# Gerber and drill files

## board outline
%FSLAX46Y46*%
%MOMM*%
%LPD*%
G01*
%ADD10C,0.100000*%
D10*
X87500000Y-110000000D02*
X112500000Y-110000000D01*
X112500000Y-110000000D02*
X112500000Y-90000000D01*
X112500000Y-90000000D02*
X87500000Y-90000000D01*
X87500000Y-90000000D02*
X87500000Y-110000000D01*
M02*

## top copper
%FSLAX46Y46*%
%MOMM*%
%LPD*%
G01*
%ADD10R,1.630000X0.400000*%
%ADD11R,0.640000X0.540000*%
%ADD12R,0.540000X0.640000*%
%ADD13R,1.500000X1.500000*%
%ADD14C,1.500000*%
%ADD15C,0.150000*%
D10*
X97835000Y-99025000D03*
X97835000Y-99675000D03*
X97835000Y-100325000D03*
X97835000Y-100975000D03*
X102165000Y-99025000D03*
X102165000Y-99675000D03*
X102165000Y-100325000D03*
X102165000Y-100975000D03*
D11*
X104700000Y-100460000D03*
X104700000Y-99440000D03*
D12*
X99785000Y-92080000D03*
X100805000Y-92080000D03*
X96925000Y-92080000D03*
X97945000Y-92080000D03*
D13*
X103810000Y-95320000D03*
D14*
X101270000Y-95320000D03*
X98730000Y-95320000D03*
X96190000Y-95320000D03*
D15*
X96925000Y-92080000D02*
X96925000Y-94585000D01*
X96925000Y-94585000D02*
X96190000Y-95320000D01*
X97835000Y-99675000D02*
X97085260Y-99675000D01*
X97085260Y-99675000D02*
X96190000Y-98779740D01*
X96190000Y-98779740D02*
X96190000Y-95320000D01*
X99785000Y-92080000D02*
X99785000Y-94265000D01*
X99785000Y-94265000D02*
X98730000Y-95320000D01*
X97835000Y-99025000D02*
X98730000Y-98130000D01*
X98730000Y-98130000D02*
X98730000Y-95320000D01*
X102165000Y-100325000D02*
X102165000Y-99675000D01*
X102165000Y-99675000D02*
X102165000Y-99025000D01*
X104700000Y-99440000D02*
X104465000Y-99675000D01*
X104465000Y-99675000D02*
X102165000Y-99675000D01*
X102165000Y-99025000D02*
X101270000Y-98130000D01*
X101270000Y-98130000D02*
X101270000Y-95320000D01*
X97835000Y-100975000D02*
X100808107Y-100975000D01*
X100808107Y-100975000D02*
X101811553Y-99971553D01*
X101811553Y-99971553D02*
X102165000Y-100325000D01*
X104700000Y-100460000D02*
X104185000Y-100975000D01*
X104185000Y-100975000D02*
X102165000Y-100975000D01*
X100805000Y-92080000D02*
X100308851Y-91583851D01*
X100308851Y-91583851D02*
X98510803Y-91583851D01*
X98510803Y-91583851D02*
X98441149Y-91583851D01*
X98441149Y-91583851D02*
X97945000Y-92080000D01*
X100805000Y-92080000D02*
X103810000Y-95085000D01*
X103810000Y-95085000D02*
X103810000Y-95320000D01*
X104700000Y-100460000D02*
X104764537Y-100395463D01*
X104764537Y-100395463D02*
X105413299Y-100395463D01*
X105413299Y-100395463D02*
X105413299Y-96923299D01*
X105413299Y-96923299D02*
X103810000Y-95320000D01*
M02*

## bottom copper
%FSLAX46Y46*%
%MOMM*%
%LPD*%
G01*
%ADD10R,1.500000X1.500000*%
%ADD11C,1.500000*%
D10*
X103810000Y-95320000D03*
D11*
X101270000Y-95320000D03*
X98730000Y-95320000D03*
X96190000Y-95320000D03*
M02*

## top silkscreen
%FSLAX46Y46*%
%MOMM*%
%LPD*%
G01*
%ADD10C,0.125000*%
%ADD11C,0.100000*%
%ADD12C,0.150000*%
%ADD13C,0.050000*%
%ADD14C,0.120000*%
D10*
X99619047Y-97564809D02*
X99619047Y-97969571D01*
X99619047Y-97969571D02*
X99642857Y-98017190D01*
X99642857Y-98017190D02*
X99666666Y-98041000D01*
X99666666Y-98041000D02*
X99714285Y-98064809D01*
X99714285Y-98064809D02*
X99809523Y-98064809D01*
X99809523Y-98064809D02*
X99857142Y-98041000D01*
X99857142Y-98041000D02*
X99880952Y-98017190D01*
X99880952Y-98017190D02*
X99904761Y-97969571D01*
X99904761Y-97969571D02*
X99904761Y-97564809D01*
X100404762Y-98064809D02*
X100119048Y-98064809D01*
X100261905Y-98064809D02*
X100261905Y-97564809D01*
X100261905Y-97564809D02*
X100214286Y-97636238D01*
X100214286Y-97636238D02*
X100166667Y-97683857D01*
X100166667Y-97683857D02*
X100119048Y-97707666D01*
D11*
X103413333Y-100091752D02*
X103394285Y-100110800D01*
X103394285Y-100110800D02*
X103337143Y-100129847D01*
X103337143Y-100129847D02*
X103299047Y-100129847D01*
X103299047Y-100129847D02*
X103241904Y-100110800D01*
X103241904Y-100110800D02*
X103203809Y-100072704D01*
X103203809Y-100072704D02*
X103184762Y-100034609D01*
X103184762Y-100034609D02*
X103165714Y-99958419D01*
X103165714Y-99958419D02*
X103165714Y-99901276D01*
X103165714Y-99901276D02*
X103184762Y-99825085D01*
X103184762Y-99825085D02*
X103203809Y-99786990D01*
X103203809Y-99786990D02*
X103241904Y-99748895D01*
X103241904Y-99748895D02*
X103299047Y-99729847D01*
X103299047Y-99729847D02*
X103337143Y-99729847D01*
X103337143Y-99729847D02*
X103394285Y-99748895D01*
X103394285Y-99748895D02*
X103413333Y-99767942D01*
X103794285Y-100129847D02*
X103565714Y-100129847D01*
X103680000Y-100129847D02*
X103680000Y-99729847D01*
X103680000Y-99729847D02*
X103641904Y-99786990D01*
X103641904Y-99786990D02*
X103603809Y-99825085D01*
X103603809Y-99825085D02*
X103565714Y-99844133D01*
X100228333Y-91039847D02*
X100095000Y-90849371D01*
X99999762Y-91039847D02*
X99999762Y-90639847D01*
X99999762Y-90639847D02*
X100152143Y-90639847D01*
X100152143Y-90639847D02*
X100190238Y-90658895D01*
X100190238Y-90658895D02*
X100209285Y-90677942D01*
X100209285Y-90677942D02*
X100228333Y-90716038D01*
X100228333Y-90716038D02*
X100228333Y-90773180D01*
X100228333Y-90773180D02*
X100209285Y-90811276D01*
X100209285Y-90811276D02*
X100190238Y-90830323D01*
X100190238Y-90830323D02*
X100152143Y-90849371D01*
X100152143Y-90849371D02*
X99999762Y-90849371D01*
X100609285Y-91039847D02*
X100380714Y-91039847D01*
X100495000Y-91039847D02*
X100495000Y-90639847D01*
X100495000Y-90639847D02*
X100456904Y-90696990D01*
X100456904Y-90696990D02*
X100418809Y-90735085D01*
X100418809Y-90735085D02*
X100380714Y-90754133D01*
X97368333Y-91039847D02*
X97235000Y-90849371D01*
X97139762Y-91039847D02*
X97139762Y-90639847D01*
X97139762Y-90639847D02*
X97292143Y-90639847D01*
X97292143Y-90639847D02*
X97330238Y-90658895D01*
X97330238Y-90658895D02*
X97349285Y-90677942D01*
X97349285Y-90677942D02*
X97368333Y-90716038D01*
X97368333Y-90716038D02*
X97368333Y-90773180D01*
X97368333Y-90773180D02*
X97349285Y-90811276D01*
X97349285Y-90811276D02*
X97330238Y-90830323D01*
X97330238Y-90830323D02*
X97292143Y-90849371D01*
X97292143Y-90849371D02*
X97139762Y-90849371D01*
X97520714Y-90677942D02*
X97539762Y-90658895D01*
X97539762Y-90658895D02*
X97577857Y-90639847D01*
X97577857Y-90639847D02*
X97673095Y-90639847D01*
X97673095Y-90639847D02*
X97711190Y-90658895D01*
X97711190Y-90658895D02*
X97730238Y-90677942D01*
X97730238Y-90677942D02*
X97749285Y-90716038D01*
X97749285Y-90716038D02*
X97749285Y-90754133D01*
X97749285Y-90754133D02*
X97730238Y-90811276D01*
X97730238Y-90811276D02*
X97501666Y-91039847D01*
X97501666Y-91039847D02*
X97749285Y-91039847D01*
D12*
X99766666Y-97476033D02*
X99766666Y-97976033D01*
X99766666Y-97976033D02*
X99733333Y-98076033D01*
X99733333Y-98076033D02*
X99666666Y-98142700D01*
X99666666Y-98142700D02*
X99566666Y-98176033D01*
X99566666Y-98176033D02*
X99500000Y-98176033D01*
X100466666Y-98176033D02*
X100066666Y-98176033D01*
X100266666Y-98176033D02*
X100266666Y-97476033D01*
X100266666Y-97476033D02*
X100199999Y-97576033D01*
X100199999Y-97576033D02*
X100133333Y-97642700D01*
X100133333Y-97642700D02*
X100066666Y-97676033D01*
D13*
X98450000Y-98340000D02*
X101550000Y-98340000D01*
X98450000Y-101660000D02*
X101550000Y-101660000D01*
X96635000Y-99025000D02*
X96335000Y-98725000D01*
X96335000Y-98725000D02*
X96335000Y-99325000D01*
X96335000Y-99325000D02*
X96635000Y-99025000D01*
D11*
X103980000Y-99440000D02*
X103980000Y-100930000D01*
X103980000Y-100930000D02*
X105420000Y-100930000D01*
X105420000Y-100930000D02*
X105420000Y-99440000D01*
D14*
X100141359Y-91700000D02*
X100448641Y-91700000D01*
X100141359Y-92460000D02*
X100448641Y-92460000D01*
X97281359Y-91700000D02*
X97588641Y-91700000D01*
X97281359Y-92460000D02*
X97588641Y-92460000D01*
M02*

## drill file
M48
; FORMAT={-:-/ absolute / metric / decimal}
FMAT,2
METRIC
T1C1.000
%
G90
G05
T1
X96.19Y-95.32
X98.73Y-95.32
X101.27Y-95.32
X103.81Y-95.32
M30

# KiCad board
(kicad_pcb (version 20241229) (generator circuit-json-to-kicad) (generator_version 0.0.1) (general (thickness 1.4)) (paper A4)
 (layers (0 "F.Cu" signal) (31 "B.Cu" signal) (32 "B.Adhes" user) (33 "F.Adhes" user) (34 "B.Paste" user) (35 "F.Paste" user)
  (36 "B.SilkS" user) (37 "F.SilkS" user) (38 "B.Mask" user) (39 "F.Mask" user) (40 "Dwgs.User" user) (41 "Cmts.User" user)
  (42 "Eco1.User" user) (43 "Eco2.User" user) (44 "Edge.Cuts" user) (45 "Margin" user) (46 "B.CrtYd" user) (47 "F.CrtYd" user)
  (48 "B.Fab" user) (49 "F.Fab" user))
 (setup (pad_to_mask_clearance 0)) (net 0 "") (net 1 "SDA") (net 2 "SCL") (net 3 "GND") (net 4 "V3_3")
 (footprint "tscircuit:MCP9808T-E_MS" (layer F.Cu) (at 100 100 0)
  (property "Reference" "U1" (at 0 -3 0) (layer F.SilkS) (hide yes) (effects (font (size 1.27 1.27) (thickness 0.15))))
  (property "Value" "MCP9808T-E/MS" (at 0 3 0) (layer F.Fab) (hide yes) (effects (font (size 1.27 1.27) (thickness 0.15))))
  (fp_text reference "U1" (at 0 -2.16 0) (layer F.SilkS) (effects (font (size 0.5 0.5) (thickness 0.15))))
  (fp_line (start -1.55 -1.66) (end 1.55 -1.66) (stroke (width 0.05) (type default)) (layer F.SilkS))
  (fp_line (start -1.55 1.66) (end 1.55 1.66) (stroke (width 0.05) (type default)) (layer F.SilkS))
  (fp_line (start -3.3649999999999998 -0.9750000000000001) (end -3.665 -1.2750000000000001) (stroke (width 0.05) (type default))
   (layer F.SilkS))
  (fp_line (start -3.665 -1.2750000000000001) (end -3.665 -0.675) (stroke (width 0.05) (type default)) (layer F.SilkS))
  (fp_line (start -3.665 -0.675) (end -3.3649999999999998 -0.9750000000000001) (stroke (width 0.05) (type default)) (layer F.SilkS))
  (pad "1" smd rect (at -2.165 -0.9750000000000001 0) (size 1.63 0.4) (layers F.Cu F.Paste F.Mask) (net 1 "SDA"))
  (pad "2" smd rect (at -2.165 -0.325 0) (size 1.63 0.4) (layers F.Cu F.Paste F.Mask) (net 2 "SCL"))
  (pad "3" smd rect (at -2.165 0.325 0) (size 1.63 0.4) (layers F.Cu F.Paste F.Mask))
  (pad "4" smd rect (at -2.165 0.9750000000000001 0) (size 1.63 0.4) (layers F.Cu F.Paste F.Mask) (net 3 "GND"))
  (pad "5" smd rect (at 2.165 -0.9750000000000001 0) (size 1.63 0.4) (layers F.Cu F.Paste F.Mask) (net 3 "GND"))
  (pad "6" smd rect (at 2.165 -0.325 0) (size 1.63 0.4) (layers F.Cu F.Paste F.Mask) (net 3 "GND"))
  (pad "7" smd rect (at 2.165 0.325 0) (size 1.63 0.4) (layers F.Cu F.Paste F.Mask) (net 3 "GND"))
  (pad "8" smd rect (at 2.165 0.9750000000000001 0) (size 1.63 0.4) (layers F.Cu F.Paste F.Mask) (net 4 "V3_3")))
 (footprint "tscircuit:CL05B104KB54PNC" (layer F.Cu) (at 104.7 99.95 90)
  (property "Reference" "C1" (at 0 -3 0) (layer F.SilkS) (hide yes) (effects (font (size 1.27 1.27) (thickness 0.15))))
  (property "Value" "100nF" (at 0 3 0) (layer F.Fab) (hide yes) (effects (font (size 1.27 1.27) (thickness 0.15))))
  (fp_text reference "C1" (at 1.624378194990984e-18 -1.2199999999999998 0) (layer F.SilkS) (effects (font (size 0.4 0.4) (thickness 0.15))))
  (fp_line (start 0.51 -0.7199999999999998) (end -0.98 -0.7200000000000001) (stroke (width 0.1) (type default)) (layer F.SilkS))
  (fp_line (start -0.98 -0.7200000000000001) (end -0.98 0.7199999999999999) (stroke (width 0.1) (type default)) (layer F.SilkS))
  (fp_line (start -0.98 0.7199999999999999) (end 0.51 0.7199999999999998) (stroke (width 0.1) (type default)) (layer F.SilkS))
  (pad "1" smd rect (at -0.51 0 0) (size 0.64 0.54) (layers F.Cu F.Paste F.Mask) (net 4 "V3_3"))
  (pad "2" smd rect (at 0.51 0 0) (size 0.64 0.54) (layers F.Cu F.Paste F.Mask) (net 3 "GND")))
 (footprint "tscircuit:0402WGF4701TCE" (layer F.Cu) (at 100.295 92.08 0)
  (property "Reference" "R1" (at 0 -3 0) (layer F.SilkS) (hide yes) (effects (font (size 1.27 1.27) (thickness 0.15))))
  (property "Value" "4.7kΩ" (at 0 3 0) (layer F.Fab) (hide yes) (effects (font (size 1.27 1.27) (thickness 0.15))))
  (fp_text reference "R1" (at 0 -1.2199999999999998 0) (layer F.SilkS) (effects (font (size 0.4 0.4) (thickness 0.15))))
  (fp_line (start -0.153641 -0.3799999999999999) (end 0.15364100000000003 -0.3799999999999999) (stroke (width 0.12) (type default))
   (layer F.SilkS))
  (fp_line (start -0.153641 0.3799999999999999) (end 0.15364100000000003 0.3799999999999999) (stroke (width 0.12) (type default))
   (layer F.SilkS))
  (pad "1" smd rect (at -0.51 0 0) (size 0.54 0.64) (layers F.Cu F.Paste F.Mask) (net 1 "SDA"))
  (pad "2" smd rect (at 0.51 0 0) (size 0.54 0.64) (layers F.Cu F.Paste F.Mask) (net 4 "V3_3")))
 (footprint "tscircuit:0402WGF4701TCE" (layer F.Cu) (at 97.435 92.08 0)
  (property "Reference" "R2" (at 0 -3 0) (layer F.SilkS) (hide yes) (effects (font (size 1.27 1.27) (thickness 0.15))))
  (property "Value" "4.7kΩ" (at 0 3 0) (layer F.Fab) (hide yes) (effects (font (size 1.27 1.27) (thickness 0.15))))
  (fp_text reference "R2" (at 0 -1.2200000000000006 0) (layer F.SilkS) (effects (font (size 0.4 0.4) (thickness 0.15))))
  (fp_line (start -0.15364099999999992 -0.3800000000000008) (end 0.15364099999999992 -0.3800000000000008)
   (stroke (width 0.12) (type default)) (layer F.SilkS))
  (fp_line (start -0.15364099999999992 0.3799999999999999) (end 0.15364099999999992 0.3799999999999999) (stroke (width 0.12) (type default))
   (layer F.SilkS))
  (pad "1" smd rect (at -0.5099999999999998 0 0) (size 0.54 0.64) (layers F.Cu F.Paste F.Mask) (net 2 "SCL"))
  (pad "2" smd rect (at 0.5099999999999998 0 0) (size 0.54 0.64) (layers F.Cu F.Paste F.Mask) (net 4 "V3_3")))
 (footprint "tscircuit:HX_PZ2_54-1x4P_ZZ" (layer F.Cu) (at 100 95.32 180)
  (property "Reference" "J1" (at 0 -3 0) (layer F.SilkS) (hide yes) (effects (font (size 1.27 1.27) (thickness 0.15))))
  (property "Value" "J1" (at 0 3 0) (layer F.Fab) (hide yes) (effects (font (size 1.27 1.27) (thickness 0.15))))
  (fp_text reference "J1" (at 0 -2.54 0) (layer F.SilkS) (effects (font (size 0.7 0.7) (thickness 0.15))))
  (pad "1" thru_hole rect (at -3.81 -4.215879892249837e-16 0) (size 1.5 1.5) (drill 1) (layers *.Cu *.Mask) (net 4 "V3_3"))
  (pad "2" thru_hole circle (at -1.27 1.5553014349171386e-16 0) (size 1.5 1.5) (drill 1) (layers *.Cu *.Mask) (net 3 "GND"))
  (pad "3" thru_hole circle (at 1.27 -1.5553014349171386e-16 0) (size 1.5 1.5) (drill 1) (layers *.Cu *.Mask) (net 1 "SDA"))
  (pad "4" thru_hole circle (at 3.81 4.215879892249837e-16 0) (size 1.5 1.5) (drill 1) (layers *.Cu *.Mask) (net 2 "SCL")))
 (segment (start 96.925 92.08) (end 96.925 94.58500000000001) (width 0.15) (layer F.Cu) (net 2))
 (segment (start 96.925 94.58500000000001) (end 96.19 95.32) (width 0.15) (layer F.Cu) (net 2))
 (segment (start 97.835 99.675) (end 97.08525987884752 99.675) (width 0.15) (layer F.Cu) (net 2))
 (segment (start 97.08525987884752 99.675) (end 96.19 98.77974012115249) (width 0.15) (layer F.Cu) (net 2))
 (segment (start 96.19 98.77974012115249) (end 96.19 95.32) (width 0.15) (layer F.Cu) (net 2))
 (segment (start 99.785 92.08) (end 99.785 94.265) (width 0.15) (layer F.Cu) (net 1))
 (segment (start 99.785 94.265) (end 98.73 95.32) (width 0.15) (layer F.Cu) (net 1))
 (segment (start 97.835 99.025) (end 98.73 98.13) (width 0.15) (layer F.Cu) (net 1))
 (segment (start 98.73 98.13) (end 98.73 95.32) (width 0.15) (layer F.Cu) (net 1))
 (segment (start 102.165 100.325) (end 102.165 99.675) (width 0.15) (layer F.Cu) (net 3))
 (segment (start 102.165 99.675) (end 102.165 99.025) (width 0.15) (layer F.Cu) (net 3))
 (segment (start 104.7 99.44) (end 104.465 99.675) (width 0.15) (layer F.Cu) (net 3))
 (segment (start 104.465 99.675) (end 102.165 99.675) (width 0.15) (layer F.Cu) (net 3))
 (segment (start 102.165 99.025) (end 101.27 98.13) (width 0.15) (layer F.Cu) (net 3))
 (segment (start 101.27 98.13) (end 101.27 95.32) (width 0.15) (layer F.Cu) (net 3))
 (segment (start 97.835 100.975) (end 100.80810689301062 100.975) (width 0.15) (layer F.Cu) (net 3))
 (segment (start 100.80810689301062 100.975) (end 101.81155344650531 99.97155344650531) (width 0.15) (layer F.Cu) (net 3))
 (segment (start 101.81155344650531 99.97155344650531) (end 102.165 100.325) (width 0.15) (layer F.Cu) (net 3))
 (segment (start 104.7 100.46) (end 104.185 100.975) (width 0.15) (layer F.Cu) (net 4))
 (segment (start 104.185 100.975) (end 102.165 100.975) (width 0.15) (layer F.Cu) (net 4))
 (segment (start 100.80499999999999 92.08) (end 100.30885116143016 91.58385116143016) (width 0.15) (layer F.Cu) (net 4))
 (segment (start 100.30885116143016 91.58385116143016) (end 98.5108025811472 91.58385116143016) (width 0.15) (layer F.Cu) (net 4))
 (segment (start 98.5108025811472 91.58385116143016) (end 98.44114883856984 91.58385116143016) (width 0.15) (layer F.Cu) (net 4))
 (segment (start 98.44114883856984 91.58385116143016) (end 97.945 92.08) (width 0.15) (layer F.Cu) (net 4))
 (segment (start 100.80499999999999 92.08) (end 103.81 95.08500000000001) (width 0.15) (layer F.Cu) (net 4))
 (segment (start 103.81 95.08500000000001) (end 103.81 95.32) (width 0.15) (layer F.Cu) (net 4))
 (segment (start 104.7 100.46) (end 104.76453745293394 100.39546254706606) (width 0.15) (layer F.Cu) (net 4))
 (segment (start 104.76453745293394 100.39546254706606) (end 105.41329870445198 100.39546254706606) (width 0.15) (layer F.Cu) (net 4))
 (segment (start 105.41329870445198 100.39546254706606) (end 105.41329870445198 96.92329870445198) (width 0.15) (layer F.Cu) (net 4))
 (segment (start 105.41329870445198 96.92329870445198) (end 103.81 95.32) (width 0.15) (layer F.Cu) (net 4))
 (gr_line (start 87.5 110) (end 112.5 110) (width 0.1) (layer Edge.Cuts))
 (gr_line (start 112.5 110) (end 112.5 90) (width 0.1) (layer Edge.Cuts))
 (gr_line (start 112.5 90) (end 87.5 90) (width 0.1) (layer Edge.Cuts))
 (gr_line (start 87.5 90) (end 87.5 110) (width 0.1) (layer Edge.Cuts)))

